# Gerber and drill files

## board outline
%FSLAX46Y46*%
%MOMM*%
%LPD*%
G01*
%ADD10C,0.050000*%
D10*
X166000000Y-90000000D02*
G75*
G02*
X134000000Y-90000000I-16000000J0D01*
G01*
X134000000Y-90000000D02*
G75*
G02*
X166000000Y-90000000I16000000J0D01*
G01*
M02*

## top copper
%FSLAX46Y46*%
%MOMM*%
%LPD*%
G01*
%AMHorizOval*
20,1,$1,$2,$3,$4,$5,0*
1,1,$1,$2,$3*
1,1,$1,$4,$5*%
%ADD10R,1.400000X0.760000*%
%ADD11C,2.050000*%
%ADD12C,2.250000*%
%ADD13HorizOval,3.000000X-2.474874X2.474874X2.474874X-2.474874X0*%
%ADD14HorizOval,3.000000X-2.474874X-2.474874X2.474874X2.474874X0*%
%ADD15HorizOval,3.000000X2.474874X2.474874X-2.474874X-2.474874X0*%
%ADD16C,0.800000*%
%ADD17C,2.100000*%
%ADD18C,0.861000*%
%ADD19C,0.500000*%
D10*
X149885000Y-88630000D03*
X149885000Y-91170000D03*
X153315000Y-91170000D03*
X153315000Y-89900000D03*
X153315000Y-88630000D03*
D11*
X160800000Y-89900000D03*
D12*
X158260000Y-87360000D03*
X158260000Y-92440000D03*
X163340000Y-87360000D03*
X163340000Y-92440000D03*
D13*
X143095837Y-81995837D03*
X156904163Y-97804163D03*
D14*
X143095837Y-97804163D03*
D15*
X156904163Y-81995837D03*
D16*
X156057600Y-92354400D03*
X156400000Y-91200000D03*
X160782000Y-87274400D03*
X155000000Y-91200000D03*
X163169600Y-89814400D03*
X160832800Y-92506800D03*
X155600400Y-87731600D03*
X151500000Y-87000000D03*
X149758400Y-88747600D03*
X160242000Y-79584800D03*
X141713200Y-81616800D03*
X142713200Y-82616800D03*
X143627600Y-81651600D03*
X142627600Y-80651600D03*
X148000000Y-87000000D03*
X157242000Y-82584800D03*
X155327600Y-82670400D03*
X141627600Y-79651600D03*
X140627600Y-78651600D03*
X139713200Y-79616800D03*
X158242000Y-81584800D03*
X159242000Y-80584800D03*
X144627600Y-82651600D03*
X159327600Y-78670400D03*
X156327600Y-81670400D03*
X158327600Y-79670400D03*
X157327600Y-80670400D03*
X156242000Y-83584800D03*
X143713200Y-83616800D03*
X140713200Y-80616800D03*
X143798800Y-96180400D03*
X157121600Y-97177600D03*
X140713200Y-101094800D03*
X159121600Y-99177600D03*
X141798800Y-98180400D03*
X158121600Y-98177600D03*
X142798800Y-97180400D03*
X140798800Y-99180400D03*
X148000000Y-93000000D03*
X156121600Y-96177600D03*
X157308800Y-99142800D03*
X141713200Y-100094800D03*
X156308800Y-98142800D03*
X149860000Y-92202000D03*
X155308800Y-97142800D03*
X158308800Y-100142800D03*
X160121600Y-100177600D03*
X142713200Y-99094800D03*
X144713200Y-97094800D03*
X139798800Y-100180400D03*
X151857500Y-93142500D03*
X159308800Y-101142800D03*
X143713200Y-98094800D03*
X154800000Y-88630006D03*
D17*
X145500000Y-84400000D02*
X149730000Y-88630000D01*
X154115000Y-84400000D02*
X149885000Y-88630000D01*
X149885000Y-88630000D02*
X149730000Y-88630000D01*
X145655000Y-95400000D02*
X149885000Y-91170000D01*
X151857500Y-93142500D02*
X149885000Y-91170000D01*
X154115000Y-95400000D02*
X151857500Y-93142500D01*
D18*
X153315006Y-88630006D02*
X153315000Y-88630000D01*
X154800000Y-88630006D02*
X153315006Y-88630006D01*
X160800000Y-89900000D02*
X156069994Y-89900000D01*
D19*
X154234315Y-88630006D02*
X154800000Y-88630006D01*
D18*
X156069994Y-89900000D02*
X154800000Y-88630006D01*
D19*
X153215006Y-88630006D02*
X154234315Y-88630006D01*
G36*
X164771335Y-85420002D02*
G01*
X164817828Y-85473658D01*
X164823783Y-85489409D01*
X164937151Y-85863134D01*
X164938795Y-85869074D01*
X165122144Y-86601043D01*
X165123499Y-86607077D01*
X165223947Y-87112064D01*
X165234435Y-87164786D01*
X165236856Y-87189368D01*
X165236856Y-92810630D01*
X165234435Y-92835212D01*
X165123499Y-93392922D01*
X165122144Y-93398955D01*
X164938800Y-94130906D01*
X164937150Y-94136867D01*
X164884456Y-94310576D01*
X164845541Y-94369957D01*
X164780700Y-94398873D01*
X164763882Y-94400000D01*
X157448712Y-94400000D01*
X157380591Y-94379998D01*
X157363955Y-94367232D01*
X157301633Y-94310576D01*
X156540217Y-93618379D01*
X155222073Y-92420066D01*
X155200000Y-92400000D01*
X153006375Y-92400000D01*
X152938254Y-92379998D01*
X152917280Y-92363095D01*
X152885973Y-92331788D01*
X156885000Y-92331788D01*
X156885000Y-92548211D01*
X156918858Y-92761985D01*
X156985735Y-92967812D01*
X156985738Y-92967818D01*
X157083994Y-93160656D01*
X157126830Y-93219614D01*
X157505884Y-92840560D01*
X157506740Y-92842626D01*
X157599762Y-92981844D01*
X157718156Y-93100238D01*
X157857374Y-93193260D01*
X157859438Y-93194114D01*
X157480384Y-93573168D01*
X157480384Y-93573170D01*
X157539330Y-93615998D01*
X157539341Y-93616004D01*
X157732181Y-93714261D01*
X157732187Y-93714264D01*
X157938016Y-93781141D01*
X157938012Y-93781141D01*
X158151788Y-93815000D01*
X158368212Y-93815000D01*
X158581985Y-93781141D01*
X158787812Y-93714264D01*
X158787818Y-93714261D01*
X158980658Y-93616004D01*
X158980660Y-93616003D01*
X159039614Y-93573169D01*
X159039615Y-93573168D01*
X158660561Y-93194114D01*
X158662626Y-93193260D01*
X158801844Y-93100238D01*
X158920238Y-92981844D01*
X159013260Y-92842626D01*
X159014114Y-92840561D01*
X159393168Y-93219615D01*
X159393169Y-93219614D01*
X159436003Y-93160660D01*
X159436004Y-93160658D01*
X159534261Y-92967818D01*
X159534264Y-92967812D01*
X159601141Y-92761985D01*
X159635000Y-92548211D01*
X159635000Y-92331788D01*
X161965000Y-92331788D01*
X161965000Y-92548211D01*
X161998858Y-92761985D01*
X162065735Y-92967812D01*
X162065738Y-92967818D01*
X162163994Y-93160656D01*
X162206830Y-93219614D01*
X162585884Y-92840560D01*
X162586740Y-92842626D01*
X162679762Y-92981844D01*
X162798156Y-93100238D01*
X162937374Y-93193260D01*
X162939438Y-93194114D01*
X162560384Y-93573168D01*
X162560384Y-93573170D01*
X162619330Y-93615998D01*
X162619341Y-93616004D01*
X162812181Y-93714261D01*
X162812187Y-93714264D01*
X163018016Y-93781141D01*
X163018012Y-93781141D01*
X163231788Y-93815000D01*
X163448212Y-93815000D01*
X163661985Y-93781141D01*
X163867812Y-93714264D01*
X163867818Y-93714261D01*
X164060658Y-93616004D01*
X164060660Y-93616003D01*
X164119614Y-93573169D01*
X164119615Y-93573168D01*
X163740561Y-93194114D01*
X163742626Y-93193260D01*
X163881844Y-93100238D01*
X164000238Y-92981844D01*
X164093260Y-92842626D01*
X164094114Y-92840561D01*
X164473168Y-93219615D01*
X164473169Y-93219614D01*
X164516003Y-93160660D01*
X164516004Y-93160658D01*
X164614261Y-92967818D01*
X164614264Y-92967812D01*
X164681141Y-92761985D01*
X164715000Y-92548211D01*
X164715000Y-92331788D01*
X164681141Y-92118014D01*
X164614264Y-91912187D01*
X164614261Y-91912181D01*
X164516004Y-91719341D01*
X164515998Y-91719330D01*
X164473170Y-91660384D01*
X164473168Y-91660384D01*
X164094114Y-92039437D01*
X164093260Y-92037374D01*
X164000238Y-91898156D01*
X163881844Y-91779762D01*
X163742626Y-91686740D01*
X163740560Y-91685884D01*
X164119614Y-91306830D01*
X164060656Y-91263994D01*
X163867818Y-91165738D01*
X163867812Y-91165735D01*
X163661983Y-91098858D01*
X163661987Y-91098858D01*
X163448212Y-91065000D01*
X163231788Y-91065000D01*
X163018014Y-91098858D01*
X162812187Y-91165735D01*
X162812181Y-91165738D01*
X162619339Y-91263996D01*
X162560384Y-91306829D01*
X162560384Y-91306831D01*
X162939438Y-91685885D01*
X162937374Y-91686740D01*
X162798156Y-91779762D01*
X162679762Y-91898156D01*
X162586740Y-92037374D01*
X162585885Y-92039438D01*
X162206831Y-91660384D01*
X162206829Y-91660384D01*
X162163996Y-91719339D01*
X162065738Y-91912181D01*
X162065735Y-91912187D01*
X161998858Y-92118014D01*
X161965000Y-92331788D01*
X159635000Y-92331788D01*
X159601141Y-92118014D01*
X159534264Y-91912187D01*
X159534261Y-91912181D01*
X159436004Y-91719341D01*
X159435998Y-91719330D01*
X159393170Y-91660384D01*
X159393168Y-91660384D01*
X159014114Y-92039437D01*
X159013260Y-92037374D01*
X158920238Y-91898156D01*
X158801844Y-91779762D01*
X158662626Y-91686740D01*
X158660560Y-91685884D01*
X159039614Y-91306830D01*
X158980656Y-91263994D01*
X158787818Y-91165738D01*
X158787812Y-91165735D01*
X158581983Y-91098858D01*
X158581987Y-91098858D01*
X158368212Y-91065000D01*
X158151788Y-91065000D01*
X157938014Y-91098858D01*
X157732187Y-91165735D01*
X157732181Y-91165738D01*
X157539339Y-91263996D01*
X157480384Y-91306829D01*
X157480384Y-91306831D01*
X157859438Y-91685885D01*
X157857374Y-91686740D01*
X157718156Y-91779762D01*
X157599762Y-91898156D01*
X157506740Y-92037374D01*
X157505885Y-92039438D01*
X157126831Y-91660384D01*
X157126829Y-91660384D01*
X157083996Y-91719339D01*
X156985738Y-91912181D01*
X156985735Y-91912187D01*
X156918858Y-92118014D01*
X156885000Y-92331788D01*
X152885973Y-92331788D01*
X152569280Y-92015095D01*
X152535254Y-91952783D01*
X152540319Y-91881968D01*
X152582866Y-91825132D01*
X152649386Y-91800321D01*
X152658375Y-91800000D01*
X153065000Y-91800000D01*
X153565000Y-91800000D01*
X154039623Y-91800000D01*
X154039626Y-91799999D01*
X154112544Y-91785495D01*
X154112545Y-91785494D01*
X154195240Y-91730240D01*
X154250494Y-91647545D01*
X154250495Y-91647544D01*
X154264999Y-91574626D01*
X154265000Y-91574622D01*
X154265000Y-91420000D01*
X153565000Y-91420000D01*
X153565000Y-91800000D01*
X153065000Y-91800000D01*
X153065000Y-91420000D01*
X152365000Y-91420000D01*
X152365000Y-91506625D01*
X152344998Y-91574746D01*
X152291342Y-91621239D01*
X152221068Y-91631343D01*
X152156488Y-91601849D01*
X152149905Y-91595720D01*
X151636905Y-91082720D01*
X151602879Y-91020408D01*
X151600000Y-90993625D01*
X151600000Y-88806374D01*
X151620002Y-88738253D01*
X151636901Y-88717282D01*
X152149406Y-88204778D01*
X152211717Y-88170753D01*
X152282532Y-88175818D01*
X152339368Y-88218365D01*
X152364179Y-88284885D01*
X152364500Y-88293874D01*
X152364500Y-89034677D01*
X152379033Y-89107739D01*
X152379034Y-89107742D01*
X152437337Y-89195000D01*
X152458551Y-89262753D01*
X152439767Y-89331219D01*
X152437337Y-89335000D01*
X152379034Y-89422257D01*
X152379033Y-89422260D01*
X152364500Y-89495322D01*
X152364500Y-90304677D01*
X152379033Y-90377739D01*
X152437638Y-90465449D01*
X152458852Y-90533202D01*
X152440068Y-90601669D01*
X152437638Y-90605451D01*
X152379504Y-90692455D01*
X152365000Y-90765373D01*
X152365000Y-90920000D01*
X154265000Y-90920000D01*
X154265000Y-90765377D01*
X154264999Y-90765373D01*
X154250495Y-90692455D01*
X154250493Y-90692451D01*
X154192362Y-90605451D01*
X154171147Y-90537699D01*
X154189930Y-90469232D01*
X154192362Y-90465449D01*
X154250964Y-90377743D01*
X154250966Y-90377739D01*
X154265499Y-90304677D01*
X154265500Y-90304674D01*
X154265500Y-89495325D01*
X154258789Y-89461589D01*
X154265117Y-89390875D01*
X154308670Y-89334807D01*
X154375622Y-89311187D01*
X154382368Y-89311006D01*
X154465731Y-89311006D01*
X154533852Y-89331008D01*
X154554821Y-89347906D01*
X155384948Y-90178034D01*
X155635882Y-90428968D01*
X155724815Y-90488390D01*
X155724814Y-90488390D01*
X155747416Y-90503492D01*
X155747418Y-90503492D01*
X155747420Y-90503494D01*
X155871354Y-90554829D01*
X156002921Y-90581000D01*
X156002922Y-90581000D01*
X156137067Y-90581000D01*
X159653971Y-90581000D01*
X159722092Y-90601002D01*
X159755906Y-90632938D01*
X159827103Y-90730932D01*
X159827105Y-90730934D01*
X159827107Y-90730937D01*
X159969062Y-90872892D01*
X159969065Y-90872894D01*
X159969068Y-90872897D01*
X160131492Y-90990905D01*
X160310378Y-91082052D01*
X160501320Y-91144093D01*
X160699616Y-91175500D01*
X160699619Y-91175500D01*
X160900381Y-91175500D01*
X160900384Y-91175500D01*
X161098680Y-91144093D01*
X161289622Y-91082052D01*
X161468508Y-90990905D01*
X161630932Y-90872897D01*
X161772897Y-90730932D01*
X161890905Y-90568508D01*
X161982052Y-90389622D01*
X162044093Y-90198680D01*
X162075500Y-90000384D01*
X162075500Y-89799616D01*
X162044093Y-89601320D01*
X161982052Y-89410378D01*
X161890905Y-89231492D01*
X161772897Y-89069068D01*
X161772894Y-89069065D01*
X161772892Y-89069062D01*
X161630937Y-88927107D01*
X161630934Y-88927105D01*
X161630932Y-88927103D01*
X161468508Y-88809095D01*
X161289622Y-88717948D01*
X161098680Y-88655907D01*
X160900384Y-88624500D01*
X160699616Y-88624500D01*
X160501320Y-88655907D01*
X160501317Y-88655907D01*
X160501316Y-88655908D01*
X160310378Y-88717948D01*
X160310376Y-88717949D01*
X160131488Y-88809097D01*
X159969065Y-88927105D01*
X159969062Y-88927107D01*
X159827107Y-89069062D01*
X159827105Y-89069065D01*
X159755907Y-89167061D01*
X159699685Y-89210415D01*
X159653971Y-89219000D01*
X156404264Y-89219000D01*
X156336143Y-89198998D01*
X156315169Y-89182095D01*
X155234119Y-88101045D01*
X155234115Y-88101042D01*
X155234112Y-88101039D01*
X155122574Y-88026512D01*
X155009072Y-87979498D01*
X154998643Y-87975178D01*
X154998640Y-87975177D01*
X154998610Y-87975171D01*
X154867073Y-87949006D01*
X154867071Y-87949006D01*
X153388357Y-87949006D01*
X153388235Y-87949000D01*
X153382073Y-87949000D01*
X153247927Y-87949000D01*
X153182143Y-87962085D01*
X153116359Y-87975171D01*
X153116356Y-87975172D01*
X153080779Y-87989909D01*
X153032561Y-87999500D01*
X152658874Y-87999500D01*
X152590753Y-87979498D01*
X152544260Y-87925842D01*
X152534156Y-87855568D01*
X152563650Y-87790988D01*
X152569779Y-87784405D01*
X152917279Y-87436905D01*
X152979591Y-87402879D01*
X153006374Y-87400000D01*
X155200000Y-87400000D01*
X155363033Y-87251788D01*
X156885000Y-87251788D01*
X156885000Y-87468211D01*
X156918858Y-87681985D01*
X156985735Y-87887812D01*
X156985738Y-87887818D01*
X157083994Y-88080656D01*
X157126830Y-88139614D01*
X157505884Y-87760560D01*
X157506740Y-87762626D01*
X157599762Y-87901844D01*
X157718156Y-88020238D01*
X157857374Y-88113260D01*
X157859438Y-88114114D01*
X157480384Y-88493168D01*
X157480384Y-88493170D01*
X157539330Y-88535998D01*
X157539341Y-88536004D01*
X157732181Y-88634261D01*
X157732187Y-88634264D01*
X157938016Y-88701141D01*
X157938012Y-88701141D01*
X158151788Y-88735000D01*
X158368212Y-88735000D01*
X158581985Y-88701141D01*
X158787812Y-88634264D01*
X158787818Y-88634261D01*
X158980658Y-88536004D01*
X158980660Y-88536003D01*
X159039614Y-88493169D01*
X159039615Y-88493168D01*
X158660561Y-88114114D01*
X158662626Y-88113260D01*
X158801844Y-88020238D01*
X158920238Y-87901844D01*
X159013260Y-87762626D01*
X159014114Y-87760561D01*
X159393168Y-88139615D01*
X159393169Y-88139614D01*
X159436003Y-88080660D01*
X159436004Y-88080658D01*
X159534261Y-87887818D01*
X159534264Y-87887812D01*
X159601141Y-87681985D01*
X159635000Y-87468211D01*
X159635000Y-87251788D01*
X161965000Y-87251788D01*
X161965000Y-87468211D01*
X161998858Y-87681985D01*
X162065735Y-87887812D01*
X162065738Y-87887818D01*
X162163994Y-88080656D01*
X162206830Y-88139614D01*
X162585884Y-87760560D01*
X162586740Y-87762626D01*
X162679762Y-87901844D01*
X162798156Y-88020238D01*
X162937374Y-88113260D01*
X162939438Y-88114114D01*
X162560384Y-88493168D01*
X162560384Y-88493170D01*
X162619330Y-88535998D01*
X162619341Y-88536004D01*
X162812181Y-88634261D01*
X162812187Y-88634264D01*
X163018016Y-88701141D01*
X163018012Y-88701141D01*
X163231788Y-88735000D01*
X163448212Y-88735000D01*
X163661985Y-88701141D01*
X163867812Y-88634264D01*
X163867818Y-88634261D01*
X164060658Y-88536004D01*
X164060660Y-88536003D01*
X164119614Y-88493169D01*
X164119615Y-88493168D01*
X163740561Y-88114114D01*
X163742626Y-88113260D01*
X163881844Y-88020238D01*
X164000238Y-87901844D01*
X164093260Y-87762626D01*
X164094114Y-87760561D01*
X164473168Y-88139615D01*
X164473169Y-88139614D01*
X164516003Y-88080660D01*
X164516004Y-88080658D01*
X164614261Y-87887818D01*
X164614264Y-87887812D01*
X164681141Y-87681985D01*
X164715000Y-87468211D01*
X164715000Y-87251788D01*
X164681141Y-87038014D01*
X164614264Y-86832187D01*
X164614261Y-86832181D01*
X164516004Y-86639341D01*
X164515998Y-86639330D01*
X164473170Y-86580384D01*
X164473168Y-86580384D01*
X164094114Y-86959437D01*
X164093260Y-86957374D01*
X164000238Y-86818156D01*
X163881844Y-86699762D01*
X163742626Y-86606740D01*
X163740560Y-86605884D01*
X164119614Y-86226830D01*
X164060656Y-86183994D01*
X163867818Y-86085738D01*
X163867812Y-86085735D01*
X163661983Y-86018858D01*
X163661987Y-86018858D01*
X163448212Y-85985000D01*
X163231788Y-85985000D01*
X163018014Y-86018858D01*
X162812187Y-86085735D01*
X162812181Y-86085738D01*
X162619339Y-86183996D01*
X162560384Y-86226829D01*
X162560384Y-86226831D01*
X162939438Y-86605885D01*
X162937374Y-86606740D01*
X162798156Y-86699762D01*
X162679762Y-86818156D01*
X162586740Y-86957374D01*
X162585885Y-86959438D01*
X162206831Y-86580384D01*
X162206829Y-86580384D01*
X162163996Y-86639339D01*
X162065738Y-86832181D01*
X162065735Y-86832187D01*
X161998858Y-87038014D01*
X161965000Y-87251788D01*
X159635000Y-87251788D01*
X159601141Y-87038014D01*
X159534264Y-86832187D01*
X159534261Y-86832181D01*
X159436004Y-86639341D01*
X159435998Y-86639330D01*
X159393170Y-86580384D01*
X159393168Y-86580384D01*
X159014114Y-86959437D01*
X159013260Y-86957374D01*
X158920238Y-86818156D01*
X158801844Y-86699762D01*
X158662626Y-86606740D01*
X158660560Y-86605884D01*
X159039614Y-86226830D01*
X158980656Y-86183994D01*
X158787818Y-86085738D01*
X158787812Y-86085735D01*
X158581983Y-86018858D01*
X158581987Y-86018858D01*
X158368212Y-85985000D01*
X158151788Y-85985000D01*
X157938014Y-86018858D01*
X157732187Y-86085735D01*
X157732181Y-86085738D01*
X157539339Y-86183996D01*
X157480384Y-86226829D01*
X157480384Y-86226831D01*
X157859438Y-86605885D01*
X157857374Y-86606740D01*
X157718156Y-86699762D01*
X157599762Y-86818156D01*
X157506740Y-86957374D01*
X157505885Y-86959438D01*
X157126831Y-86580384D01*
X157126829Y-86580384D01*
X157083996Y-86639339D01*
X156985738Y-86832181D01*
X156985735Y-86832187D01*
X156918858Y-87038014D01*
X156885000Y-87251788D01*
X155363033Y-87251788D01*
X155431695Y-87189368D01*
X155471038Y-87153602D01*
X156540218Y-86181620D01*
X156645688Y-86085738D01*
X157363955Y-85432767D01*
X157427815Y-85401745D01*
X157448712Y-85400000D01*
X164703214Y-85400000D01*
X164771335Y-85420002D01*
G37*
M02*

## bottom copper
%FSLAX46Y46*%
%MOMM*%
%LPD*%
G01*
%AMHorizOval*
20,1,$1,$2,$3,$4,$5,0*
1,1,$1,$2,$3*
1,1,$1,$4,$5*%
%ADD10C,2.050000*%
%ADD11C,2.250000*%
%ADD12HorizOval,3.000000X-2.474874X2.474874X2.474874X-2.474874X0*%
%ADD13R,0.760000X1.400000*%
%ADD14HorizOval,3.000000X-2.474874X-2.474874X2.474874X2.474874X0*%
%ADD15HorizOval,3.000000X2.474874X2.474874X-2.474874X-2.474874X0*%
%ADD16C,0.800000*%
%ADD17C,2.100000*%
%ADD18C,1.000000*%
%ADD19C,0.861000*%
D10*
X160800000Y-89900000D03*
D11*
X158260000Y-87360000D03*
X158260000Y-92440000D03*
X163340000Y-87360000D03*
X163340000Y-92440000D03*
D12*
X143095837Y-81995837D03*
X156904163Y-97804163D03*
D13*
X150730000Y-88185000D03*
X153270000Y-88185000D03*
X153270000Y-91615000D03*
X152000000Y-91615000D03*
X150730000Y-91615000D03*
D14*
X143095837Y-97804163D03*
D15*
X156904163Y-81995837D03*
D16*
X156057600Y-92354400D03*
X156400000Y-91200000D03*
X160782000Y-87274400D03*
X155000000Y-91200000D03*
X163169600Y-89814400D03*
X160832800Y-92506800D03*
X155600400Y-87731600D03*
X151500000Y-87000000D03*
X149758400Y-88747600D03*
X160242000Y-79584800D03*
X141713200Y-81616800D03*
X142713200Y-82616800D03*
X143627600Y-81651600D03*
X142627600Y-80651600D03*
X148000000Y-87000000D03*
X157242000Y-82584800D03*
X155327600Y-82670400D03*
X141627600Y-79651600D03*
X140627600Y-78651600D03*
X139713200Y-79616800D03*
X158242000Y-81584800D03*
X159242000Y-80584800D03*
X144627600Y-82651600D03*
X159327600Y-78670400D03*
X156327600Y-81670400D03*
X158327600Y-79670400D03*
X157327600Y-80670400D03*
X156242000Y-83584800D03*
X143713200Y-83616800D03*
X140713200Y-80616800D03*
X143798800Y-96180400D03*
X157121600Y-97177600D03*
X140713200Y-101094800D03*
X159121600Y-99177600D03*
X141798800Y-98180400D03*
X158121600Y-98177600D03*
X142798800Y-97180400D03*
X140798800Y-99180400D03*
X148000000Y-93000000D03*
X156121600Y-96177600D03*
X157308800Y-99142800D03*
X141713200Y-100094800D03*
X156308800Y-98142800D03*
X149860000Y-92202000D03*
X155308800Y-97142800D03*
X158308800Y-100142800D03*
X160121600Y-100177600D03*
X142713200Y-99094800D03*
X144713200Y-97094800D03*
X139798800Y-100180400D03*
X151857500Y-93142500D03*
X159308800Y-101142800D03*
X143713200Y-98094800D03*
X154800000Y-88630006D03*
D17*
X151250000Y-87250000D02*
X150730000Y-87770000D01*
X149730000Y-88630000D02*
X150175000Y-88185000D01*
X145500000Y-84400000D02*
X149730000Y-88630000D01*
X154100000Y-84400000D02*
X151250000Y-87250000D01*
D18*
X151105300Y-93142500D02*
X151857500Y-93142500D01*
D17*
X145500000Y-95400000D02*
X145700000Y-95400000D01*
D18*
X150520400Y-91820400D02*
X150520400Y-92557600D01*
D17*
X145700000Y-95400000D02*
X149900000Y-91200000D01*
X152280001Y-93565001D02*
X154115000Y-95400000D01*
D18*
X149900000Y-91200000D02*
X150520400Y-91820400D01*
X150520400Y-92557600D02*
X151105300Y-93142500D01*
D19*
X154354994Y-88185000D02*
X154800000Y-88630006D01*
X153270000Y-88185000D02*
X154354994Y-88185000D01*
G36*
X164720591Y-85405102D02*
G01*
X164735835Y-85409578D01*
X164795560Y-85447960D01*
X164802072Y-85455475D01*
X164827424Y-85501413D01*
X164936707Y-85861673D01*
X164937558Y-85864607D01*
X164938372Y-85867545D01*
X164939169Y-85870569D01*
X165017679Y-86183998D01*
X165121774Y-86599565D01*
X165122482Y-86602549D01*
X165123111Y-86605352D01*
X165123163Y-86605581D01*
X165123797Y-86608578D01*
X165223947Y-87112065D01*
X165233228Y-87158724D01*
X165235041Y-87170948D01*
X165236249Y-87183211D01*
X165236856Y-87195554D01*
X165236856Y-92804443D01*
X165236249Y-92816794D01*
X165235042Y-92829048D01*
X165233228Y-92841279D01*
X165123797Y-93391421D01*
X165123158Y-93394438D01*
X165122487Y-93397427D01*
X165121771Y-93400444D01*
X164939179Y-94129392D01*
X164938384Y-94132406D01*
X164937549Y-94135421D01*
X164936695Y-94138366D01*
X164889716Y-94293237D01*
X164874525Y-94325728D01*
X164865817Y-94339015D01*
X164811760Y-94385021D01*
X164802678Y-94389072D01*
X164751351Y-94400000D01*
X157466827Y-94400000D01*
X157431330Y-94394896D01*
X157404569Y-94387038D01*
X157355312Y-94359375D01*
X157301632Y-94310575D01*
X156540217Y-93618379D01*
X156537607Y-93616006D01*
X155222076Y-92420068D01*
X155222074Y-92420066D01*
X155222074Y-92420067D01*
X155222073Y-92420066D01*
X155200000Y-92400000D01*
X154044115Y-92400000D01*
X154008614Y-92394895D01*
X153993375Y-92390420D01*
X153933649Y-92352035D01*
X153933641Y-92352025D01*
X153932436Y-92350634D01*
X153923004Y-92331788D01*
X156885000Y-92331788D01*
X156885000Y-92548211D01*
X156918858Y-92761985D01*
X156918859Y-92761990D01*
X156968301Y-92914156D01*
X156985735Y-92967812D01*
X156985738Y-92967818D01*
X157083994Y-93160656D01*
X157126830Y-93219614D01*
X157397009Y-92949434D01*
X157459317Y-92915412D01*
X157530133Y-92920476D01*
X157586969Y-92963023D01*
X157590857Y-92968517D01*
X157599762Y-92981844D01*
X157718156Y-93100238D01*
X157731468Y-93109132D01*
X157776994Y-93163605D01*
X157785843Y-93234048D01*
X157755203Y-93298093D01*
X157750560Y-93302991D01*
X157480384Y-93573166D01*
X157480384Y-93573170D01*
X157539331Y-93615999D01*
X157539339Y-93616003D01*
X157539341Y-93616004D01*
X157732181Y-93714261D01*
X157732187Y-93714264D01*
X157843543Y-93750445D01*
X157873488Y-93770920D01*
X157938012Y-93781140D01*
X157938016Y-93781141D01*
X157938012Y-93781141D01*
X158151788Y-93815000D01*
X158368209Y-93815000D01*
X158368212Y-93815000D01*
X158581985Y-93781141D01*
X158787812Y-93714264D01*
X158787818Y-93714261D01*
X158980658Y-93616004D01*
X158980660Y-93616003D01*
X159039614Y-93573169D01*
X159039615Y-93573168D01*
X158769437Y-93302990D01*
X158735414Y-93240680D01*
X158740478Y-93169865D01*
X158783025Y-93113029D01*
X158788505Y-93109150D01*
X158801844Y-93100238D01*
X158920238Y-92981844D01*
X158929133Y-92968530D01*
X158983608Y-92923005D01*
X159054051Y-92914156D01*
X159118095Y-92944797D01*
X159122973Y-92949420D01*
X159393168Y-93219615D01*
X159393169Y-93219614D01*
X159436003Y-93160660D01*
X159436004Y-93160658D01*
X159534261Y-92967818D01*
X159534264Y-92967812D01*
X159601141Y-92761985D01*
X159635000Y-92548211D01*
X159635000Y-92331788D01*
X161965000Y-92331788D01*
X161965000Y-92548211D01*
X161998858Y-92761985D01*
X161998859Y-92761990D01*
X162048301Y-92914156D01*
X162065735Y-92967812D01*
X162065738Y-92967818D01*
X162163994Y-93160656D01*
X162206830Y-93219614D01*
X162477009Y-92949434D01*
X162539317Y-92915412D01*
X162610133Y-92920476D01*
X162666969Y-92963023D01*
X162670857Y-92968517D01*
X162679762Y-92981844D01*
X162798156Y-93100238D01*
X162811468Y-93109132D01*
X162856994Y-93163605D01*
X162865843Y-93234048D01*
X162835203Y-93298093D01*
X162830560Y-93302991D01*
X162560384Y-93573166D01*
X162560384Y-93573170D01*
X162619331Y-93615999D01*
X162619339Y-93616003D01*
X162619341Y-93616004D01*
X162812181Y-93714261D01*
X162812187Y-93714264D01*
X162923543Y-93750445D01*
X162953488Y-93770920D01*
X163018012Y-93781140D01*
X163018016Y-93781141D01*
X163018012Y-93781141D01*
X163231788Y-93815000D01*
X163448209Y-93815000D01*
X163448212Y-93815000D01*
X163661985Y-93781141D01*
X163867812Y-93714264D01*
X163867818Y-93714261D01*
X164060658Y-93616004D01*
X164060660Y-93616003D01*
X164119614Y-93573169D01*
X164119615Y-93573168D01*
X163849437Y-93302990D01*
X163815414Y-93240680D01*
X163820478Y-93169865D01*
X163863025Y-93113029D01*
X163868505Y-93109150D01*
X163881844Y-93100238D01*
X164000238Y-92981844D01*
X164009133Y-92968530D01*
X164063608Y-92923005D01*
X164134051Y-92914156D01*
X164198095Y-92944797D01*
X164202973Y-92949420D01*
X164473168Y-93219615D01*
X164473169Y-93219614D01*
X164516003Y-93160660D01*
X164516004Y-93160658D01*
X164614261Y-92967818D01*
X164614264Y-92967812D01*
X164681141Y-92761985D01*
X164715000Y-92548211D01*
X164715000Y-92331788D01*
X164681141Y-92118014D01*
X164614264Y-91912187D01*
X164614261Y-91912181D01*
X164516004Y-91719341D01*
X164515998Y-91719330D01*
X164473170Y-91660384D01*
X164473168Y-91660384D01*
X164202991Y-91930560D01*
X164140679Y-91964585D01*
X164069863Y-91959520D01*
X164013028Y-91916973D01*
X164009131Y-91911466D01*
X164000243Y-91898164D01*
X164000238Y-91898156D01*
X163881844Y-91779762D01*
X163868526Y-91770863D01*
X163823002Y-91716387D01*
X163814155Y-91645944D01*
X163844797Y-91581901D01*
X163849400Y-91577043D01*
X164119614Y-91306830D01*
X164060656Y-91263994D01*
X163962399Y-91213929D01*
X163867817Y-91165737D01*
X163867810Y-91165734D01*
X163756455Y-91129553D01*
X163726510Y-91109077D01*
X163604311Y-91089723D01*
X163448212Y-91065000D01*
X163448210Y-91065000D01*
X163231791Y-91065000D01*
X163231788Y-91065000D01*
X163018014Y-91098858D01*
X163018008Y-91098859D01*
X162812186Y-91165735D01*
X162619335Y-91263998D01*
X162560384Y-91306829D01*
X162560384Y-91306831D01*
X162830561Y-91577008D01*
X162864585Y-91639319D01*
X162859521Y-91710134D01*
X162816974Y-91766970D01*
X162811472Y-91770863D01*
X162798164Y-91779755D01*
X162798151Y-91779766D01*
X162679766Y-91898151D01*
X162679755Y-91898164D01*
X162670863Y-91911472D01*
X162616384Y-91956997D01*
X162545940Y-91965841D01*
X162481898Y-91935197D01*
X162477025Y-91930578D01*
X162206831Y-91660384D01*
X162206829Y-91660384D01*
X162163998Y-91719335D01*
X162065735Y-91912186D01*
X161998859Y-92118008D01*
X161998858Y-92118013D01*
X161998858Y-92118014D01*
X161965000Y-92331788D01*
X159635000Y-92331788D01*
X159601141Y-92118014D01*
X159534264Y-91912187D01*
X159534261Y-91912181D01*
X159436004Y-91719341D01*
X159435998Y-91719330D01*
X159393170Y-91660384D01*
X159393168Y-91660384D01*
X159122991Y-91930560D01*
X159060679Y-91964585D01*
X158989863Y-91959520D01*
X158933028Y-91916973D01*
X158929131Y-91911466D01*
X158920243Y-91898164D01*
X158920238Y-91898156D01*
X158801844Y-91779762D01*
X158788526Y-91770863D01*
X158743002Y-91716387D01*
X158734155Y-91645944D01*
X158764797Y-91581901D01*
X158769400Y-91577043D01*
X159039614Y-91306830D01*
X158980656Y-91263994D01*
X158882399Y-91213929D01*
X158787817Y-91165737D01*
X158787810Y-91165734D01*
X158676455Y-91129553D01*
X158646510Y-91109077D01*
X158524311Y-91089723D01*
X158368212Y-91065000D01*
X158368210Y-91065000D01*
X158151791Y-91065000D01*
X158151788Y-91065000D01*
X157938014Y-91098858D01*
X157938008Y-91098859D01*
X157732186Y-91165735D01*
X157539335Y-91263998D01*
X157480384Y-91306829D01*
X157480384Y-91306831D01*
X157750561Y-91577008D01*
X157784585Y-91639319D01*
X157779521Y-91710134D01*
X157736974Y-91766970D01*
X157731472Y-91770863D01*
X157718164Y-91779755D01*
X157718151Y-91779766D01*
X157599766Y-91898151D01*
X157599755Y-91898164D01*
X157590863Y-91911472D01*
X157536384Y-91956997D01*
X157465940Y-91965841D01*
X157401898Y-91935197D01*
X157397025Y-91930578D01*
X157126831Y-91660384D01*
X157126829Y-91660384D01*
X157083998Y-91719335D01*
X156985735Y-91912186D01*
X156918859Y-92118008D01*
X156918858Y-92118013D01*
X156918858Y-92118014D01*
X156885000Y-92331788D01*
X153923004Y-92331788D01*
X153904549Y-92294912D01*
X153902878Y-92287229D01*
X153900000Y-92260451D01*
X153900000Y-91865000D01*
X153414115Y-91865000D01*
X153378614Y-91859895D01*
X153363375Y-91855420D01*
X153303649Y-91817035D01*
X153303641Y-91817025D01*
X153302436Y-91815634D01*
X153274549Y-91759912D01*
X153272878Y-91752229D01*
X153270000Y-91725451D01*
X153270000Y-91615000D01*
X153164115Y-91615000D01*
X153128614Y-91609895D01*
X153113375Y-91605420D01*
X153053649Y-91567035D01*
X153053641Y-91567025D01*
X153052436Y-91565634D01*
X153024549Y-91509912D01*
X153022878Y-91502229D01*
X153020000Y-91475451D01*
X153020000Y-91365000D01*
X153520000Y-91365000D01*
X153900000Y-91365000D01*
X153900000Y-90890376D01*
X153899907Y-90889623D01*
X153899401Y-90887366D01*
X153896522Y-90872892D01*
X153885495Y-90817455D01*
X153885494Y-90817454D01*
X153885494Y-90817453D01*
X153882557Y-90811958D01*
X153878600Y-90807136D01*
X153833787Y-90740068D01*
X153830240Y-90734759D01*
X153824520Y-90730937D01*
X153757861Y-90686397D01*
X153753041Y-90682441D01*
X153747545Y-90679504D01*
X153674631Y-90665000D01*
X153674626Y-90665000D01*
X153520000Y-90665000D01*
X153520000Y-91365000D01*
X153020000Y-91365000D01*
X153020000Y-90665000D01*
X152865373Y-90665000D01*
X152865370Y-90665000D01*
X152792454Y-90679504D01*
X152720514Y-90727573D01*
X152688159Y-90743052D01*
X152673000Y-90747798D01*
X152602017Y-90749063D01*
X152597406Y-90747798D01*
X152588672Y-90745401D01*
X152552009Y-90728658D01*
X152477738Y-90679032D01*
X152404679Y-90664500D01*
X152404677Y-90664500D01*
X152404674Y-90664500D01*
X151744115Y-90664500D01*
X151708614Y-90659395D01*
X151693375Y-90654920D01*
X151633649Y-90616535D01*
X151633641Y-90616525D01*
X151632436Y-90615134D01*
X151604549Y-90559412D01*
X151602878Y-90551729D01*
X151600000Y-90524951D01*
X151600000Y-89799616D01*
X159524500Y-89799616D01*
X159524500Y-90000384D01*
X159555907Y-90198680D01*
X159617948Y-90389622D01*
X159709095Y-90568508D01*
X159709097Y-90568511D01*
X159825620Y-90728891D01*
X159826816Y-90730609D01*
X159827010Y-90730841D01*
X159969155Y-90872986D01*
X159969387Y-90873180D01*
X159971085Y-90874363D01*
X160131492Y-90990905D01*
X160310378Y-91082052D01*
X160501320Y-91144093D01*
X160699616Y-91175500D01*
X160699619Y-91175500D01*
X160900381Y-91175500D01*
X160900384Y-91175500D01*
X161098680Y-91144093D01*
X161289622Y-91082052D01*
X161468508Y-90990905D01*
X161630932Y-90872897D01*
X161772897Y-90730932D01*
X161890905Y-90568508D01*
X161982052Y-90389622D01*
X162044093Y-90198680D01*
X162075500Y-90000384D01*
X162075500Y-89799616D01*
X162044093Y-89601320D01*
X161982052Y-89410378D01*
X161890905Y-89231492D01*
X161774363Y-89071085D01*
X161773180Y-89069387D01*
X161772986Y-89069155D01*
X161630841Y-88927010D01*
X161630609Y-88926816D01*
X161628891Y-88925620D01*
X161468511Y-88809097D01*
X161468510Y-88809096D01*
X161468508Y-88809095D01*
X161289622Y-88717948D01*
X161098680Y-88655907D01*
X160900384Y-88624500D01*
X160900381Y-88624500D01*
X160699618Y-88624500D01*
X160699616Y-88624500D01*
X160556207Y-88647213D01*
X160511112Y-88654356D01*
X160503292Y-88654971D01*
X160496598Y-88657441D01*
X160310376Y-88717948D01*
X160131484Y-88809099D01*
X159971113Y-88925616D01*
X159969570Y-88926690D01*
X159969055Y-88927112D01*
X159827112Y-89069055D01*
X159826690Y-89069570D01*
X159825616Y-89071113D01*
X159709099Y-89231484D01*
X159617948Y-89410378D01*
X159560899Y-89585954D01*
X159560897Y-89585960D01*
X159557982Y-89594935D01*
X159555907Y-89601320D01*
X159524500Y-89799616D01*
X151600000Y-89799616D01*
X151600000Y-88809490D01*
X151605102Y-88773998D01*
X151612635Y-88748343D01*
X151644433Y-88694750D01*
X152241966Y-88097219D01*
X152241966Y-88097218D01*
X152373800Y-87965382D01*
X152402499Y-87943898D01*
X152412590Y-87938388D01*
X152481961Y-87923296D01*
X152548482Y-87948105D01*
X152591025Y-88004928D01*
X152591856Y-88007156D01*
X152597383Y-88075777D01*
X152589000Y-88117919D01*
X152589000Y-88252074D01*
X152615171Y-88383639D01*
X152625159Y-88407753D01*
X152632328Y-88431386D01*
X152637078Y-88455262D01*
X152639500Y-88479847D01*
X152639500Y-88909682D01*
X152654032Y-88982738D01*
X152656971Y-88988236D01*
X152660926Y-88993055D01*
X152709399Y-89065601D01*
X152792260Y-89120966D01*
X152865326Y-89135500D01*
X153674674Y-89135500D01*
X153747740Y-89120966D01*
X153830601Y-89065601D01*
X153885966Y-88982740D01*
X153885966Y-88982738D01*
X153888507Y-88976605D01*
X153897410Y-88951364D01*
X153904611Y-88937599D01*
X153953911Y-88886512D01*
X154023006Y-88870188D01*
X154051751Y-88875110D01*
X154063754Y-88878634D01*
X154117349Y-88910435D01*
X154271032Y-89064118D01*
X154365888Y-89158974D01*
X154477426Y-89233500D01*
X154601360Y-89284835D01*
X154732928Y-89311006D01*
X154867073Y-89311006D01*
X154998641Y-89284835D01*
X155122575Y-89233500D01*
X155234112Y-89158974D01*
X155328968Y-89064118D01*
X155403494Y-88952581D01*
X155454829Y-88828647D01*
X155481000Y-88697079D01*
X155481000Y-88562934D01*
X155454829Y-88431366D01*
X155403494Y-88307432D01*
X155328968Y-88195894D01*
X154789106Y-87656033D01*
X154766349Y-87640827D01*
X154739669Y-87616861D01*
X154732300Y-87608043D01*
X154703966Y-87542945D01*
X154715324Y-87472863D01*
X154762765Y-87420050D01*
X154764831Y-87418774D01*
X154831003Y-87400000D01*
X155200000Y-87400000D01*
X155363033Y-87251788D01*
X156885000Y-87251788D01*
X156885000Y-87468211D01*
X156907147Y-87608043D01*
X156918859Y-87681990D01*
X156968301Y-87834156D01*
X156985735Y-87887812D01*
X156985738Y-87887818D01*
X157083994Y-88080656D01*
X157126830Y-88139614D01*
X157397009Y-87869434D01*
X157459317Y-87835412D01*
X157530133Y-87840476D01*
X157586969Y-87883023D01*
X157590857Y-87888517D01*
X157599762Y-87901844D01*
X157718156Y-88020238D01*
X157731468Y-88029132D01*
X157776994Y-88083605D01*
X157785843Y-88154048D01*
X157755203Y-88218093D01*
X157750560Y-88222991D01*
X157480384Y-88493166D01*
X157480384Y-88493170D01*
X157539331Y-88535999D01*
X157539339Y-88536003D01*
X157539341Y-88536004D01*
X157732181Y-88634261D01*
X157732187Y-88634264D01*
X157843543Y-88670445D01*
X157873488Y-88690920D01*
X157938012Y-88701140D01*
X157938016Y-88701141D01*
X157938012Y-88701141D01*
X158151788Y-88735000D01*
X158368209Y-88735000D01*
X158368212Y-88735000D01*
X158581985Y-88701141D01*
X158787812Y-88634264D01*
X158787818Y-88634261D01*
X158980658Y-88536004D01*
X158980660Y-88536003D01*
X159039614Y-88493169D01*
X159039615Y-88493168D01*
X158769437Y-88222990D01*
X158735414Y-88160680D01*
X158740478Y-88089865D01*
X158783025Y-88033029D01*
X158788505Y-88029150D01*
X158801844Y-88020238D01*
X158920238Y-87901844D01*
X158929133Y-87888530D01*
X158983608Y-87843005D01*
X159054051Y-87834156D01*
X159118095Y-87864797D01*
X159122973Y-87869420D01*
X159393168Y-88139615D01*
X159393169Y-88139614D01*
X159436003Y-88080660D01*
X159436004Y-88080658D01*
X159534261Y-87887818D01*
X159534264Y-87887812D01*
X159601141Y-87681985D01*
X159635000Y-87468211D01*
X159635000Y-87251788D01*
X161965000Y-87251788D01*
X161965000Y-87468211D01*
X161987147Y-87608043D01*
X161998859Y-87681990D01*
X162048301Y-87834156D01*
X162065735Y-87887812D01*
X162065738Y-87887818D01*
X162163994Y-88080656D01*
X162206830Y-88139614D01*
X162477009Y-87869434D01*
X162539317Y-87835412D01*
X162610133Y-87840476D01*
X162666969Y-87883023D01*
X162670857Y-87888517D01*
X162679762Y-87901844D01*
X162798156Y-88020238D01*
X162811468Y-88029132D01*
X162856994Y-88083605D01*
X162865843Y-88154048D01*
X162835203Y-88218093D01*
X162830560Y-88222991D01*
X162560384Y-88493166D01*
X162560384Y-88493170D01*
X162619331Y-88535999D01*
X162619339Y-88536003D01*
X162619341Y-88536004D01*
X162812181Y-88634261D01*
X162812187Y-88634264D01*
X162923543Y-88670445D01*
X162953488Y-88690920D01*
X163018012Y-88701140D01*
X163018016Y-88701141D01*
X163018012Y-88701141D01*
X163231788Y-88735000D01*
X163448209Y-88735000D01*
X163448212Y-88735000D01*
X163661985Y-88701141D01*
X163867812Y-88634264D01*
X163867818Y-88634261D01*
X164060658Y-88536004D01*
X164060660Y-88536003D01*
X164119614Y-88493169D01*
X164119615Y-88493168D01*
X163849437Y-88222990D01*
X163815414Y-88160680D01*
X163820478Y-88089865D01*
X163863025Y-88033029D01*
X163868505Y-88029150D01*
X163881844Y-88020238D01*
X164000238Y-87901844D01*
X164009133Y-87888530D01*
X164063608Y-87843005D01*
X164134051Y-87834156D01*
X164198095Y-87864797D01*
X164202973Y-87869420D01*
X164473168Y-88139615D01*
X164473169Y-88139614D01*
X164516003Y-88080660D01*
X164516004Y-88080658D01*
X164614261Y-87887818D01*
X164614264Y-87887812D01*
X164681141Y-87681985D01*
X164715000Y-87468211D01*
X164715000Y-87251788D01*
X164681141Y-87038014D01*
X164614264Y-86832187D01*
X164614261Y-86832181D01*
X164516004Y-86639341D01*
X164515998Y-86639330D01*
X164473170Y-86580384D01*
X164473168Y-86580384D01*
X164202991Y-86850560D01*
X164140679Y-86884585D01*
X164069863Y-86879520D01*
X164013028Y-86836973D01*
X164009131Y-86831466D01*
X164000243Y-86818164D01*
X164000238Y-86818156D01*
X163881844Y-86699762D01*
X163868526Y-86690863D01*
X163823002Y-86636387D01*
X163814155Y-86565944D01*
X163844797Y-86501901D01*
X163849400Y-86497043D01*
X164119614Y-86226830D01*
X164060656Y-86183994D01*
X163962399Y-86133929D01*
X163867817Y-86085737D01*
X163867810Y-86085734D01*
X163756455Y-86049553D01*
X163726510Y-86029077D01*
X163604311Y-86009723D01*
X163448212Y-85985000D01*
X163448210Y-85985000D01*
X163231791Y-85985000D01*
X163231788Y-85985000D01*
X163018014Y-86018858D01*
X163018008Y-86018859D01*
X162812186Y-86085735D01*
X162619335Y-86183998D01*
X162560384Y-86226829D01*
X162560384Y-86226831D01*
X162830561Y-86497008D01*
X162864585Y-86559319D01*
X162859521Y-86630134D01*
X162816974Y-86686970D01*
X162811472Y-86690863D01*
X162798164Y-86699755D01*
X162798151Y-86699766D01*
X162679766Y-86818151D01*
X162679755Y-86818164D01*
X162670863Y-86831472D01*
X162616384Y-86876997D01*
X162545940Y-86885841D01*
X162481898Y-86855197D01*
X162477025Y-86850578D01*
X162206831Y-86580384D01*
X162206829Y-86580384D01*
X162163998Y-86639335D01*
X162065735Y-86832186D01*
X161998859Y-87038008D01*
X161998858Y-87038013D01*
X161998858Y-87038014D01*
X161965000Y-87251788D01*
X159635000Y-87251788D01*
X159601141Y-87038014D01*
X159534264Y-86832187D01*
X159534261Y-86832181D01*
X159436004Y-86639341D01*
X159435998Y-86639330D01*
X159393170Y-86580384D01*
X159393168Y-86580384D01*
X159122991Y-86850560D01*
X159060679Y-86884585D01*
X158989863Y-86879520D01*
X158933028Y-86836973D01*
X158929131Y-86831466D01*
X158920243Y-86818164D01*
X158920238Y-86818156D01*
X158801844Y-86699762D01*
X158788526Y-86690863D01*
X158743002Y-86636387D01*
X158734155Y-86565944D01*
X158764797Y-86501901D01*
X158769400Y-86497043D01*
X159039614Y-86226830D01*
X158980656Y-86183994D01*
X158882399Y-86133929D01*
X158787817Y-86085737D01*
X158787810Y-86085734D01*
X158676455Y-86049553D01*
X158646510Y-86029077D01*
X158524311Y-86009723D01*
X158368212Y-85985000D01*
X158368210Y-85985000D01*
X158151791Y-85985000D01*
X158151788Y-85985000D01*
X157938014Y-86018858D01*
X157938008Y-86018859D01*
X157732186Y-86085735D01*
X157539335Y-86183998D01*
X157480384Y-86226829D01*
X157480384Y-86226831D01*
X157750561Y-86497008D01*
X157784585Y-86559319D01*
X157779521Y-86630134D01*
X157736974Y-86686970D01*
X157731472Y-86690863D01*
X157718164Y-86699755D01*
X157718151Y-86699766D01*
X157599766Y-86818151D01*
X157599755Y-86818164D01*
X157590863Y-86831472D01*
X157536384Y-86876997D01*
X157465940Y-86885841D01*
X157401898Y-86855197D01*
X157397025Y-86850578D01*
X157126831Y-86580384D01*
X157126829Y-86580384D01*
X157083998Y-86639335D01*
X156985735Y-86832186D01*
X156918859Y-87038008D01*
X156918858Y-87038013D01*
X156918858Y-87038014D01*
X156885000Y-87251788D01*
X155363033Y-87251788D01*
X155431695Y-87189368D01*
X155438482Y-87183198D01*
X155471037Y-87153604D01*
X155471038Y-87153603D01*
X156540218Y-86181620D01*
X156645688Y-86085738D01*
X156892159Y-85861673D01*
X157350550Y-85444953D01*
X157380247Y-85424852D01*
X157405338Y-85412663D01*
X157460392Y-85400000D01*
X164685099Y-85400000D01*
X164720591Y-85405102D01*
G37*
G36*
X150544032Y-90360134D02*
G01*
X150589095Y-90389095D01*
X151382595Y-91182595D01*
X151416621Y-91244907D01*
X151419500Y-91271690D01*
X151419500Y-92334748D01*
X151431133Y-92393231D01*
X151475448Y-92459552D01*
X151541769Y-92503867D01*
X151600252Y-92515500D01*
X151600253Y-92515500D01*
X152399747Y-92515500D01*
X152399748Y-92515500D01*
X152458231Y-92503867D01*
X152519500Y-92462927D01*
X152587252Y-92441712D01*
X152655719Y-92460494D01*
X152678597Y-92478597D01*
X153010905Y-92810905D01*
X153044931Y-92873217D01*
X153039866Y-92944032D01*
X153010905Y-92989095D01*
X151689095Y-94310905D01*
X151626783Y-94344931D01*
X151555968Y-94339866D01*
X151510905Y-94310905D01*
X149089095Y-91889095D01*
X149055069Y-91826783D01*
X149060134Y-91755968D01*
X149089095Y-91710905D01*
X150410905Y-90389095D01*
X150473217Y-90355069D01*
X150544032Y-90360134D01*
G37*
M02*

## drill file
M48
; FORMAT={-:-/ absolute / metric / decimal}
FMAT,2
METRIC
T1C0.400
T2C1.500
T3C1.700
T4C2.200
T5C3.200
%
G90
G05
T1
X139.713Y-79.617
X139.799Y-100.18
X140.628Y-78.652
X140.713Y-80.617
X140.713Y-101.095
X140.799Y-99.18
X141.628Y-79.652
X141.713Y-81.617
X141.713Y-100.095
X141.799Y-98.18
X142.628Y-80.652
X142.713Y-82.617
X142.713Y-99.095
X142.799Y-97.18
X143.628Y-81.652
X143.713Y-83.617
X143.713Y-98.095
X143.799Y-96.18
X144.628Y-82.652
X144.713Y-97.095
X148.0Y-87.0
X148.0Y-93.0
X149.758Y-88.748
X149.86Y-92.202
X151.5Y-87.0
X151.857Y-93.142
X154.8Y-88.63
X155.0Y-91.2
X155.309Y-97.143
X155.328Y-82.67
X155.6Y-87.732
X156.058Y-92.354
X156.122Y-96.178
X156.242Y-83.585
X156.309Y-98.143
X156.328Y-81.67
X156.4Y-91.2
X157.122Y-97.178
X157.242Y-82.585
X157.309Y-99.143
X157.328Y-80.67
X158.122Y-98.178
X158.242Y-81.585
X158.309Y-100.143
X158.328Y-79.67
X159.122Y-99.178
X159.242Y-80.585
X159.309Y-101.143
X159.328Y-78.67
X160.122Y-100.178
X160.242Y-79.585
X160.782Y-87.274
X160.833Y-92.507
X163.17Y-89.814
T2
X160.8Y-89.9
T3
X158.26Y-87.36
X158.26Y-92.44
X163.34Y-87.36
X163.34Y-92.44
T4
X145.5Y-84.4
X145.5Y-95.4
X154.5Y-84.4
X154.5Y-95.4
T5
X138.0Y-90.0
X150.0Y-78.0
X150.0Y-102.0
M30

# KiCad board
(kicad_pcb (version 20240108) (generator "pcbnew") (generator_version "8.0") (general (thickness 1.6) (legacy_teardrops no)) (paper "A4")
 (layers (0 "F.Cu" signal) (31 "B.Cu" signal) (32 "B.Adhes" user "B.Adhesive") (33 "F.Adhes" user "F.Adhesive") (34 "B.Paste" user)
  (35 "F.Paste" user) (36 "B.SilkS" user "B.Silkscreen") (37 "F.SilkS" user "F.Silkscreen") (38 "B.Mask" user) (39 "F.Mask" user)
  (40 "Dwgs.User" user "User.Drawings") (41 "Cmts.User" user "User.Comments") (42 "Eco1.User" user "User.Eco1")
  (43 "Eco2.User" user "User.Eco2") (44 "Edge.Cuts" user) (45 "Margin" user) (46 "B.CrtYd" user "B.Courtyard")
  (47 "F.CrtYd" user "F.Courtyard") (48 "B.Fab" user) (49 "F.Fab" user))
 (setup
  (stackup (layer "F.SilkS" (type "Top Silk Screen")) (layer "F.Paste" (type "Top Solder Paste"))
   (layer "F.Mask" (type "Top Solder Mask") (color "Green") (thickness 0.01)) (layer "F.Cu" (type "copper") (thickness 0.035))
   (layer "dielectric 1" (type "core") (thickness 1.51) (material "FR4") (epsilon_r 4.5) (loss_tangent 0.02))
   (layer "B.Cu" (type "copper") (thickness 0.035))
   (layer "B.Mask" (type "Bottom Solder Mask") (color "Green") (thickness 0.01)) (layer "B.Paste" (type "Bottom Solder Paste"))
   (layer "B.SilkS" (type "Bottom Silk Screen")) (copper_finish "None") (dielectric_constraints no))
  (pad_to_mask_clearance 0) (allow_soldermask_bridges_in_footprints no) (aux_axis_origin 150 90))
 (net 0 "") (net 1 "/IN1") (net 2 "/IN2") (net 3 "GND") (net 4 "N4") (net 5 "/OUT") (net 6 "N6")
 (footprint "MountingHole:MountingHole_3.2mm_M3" (layer "F.Cu") (at 138 90)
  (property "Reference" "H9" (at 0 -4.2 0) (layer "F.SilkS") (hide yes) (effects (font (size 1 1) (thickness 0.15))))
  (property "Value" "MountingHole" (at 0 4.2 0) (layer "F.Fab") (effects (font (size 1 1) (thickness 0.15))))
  (pad "" np_thru_hole circle (at 0 0) (size 3.2 3.2) (drill 3.2) (layers "*.Cu" "*.Mask")))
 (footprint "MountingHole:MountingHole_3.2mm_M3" (layer "F.Cu") (at 150 102)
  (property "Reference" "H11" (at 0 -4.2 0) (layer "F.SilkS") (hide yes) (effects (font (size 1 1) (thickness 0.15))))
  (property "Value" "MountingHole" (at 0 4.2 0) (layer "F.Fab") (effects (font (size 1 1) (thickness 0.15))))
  (pad "" np_thru_hole circle (at 0 0) (size 3.2 3.2) (drill 3.2) (layers "*.Cu" "*.Mask")))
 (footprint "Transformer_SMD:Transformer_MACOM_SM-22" (layer "F.Cu") (at 151.6 89.9)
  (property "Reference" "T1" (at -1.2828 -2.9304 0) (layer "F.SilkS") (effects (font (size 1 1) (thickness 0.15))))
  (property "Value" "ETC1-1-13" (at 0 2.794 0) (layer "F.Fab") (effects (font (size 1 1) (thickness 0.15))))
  (pad "1" smd rect (at -1.715 -1.27) (size 1.4 0.76) (layers "F.Cu" "F.Paste" "F.Mask") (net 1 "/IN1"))
  (pad "2" smd rect (at -1.715 1.27) (size 1.4 0.76) (layers "F.Cu" "F.Paste" "F.Mask") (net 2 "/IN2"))
  (pad "3" smd rect (at 1.715 1.27) (size 1.4 0.76) (layers "F.Cu" "F.Paste" "F.Mask") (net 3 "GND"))
  (pad "4" smd rect (at 1.715 0) (size 1.4 0.76) (layers "F.Cu" "F.Paste" "F.Mask") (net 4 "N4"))
  (pad "5" smd rect (at 1.715 -1.27) (size 1.4 0.76) (layers "F.Cu" "F.Paste" "F.Mask") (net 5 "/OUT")))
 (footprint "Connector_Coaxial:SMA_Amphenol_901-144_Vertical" (layer "F.Cu") (at 160.8 89.9)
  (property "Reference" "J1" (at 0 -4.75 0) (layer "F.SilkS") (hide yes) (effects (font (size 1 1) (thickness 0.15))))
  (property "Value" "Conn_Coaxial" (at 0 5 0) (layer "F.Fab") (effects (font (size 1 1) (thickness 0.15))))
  (pad "1" thru_hole circle (at 0 0) (size 2.05 2.05) (drill 1.5) (layers "*.Cu" "*.Mask") (remove_unused_layers no) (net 5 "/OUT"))
  (pad "2" thru_hole circle (at -2.54 -2.54) (size 2.25 2.25) (drill 1.7) (layers "*.Cu" "*.Mask") (remove_unused_layers no) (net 3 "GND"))
  (pad "2" thru_hole circle (at -2.54 2.54) (size 2.25 2.25) (drill 1.7) (layers "*.Cu" "*.Mask") (remove_unused_layers no) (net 3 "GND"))
  (pad "2" thru_hole circle (at 2.54 -2.54) (size 2.25 2.25) (drill 1.7) (layers "*.Cu" "*.Mask") (remove_unused_layers no) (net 3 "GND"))
  (pad "2" thru_hole circle (at 2.54 2.54) (size 2.25 2.25) (drill 1.7) (layers "*.Cu" "*.Mask") (remove_unused_layers no) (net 3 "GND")))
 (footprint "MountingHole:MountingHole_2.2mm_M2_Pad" (layer "F.Cu") (at 145.5 84.4)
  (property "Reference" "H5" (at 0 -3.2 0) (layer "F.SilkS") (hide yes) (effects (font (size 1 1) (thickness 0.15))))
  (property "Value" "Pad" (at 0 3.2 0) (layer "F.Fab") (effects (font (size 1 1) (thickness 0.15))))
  (pad "1" thru_hole oval (at 0 0 45) (size 3 10) (drill 2.2 (offset 0 -3.4)) (layers "*.Cu" "*.Mask") (remove_unused_layers no)
   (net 1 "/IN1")))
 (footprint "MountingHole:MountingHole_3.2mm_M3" (layer "F.Cu") (at 150 78)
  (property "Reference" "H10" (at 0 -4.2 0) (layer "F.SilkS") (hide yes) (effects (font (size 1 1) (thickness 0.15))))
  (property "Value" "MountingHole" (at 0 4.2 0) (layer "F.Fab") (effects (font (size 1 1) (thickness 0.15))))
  (pad "" np_thru_hole circle (at 0 0) (size 3.2 3.2) (drill 3.2) (layers "*.Cu" "*.Mask")))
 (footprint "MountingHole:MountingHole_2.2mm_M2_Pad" (layer "F.Cu") (at 154.5 95.4 180)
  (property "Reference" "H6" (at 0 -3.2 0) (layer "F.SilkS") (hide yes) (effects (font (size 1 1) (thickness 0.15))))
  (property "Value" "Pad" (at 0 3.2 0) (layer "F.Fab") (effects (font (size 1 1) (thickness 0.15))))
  (pad "1" thru_hole oval (at 0 0 225) (size 3 10) (drill 2.2 (offset 0 -3.4)) (layers "*.Cu" "*.Mask") (remove_unused_layers no)
   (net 2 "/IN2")))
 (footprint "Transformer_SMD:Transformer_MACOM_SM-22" (layer "B.Cu") (at 152 89.9 -90)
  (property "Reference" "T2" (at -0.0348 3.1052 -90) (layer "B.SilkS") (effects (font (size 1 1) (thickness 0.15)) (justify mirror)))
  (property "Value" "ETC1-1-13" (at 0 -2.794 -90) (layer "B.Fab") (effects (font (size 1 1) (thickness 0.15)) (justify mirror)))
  (pad "1" smd rect (at -1.715 1.27 270) (size 1.4 0.76) (layers "B.Cu" "B.Paste" "B.Mask") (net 1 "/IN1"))
  (pad "2" smd rect (at -1.715 -1.27 270) (size 1.4 0.76) (layers "B.Cu" "B.Paste" "B.Mask") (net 5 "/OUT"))
  (pad "3" smd rect (at 1.715 -1.27 270) (size 1.4 0.76) (layers "B.Cu" "B.Paste" "B.Mask") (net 3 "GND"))
  (pad "4" smd rect (at 1.715 0 270) (size 1.4 0.76) (layers "B.Cu" "B.Paste" "B.Mask") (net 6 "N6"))
  (pad "5" smd rect (at 1.715 1.27 270) (size 1.4 0.76) (layers "B.Cu" "B.Paste" "B.Mask") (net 2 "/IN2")))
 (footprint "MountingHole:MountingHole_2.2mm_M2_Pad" (layer "B.Cu") (at 145.5 95.4)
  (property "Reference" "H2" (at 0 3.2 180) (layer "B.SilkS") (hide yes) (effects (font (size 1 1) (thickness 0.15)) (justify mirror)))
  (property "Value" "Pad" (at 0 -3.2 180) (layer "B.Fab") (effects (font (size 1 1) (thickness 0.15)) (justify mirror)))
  (pad "1" thru_hole oval (at 0 0 315) (size 3 10) (drill 2.2 (offset 0 3.4)) (layers "*.Cu" "*.Mask") (remove_unused_layers no)
   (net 2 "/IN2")))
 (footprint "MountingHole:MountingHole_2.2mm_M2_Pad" (layer "B.Cu") (at 154.5 84.4 180)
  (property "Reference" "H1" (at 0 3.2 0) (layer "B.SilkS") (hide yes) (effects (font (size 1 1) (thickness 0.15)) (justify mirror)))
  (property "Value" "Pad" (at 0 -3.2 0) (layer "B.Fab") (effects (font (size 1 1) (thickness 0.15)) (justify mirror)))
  (pad "1" thru_hole oval (at 0 0 135) (size 3 10) (drill 2.2 (offset 0 3.4)) (layers "*.Cu" "*.Mask") (remove_unused_layers yes)
   (keep_end_layers no) (zone_layer_connections) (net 1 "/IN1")))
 (gr_circle (center 150 90) (end 166 90) (stroke (width 0.05) (type solid)) (fill none) (layer "Edge.Cuts"))
 (via (at 156.0576 92.3544) (size 0.8) (drill 0.4) (layers "F.Cu" "B.Cu") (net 3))
 (via (at 156.4 91.2) (size 0.8) (drill 0.4) (layers "F.Cu" "B.Cu") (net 3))
 (via (at 160.782 87.2744) (size 0.8) (drill 0.4) (layers "F.Cu" "B.Cu") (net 3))
 (via (at 155 91.2) (size 0.8) (drill 0.4) (layers "F.Cu" "B.Cu") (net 3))
 (via (at 163.1696 89.8144) (size 0.8) (drill 0.4) (layers "F.Cu" "B.Cu") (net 3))
 (via (at 160.8328 92.5068) (size 0.8) (drill 0.4) (layers "F.Cu" "B.Cu") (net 3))
 (via (at 155.6004 87.7316) (size 0.8) (drill 0.4) (layers "F.Cu" "B.Cu") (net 3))
 (segment (start 145.5 84.4) (end 149.73 88.63) (width 2.1) (layer "F.Cu") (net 1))
 (segment (start 154.115 84.4) (end 149.885 88.63) (width 2.1) (layer "F.Cu") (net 1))
 (segment (start 149.885 88.63) (end 149.73 88.63) (width 2.1) (layer "F.Cu") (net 1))
 (via (at 151.5 87) (size 0.8) (drill 0.4) (layers "F.Cu" "B.Cu") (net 1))
 (via (at 149.7584 88.7476) (size 0.8) (drill 0.4) (layers "F.Cu" "B.Cu") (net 1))
 (via (at 160.242 79.5848) (size 0.8) (drill 0.4) (layers "F.Cu" "B.Cu") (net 1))
 (via (at 141.7132 81.6168) (size 0.8) (drill 0.4) (layers "F.Cu" "B.Cu") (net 1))
 (via (at 142.7132 82.6168) (size 0.8) (drill 0.4) (layers "F.Cu" "B.Cu") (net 1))
 (via (at 143.6276 81.6516) (size 0.8) (drill 0.4) (layers "F.Cu" "B.Cu") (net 1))
 (via (at 142.6276 80.6516) (size 0.8) (drill 0.4) (layers "F.Cu" "B.Cu") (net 1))
 (via (at 148 87) (size 0.8) (drill 0.4) (layers "F.Cu" "B.Cu") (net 1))
 (via (at 157.242 82.5848) (size 0.8) (drill 0.4) (layers "F.Cu" "B.Cu") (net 1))
 (via (at 155.3276 82.6704) (size 0.8) (drill 0.4) (layers "F.Cu" "B.Cu") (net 1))
 (via (at 141.6276 79.6516) (size 0.8) (drill 0.4) (layers "F.Cu" "B.Cu") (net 1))
 (via (at 140.6276 78.6516) (size 0.8) (drill 0.4) (layers "F.Cu" "B.Cu") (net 1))
 (via (at 139.7132 79.6168) (size 0.8) (drill 0.4) (layers "F.Cu" "B.Cu") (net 1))
 (via (at 158.242 81.5848) (size 0.8) (drill 0.4) (layers "F.Cu" "B.Cu") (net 1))
 (via (at 159.242 80.5848) (size 0.8) (drill 0.4) (layers "F.Cu" "B.Cu") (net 1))
 (via (at 144.6276 82.6516) (size 0.8) (drill 0.4) (layers "F.Cu" "B.Cu") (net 1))
 (via (at 159.3276 78.6704) (size 0.8) (drill 0.4) (layers "F.Cu" "B.Cu") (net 1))
 (via (at 156.3276 81.6704) (size 0.8) (drill 0.4) (layers "F.Cu" "B.Cu") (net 1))
 (via (at 158.3276 79.6704) (size 0.8) (drill 0.4) (layers "F.Cu" "B.Cu") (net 1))
 (via (at 157.3276 80.6704) (size 0.8) (drill 0.4) (layers "F.Cu" "B.Cu") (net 1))
 (via (at 156.242 83.5848) (size 0.8) (drill 0.4) (layers "F.Cu" "B.Cu") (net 1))
 (via (at 143.7132 83.6168) (size 0.8) (drill 0.4) (layers "F.Cu" "B.Cu") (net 1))
 (via (at 140.7132 80.6168) (size 0.8) (drill 0.4) (layers "F.Cu" "B.Cu") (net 1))
 (segment (start 151.25 87.25) (end 150.73 87.77) (width 2.1) (layer "B.Cu") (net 1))
 (segment (start 149.73 88.63) (end 150.175 88.185) (width 2.1) (layer "B.Cu") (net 1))
 (segment (start 145.5 84.4) (end 149.73 88.63) (width 2.1) (layer "B.Cu") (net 1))
 (segment (start 154.1 84.4) (end 151.25 87.25) (width 2.1) (layer "B.Cu") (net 1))
 (segment (start 145.655 95.4) (end 149.885 91.17) (width 2.1) (layer "F.Cu") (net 2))
 (segment (start 151.8575 93.1425) (end 149.885 91.17) (width 2.1) (layer "F.Cu") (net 2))
 (segment (start 154.115 95.4) (end 151.8575 93.1425) (width 2.1) (layer "F.Cu") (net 2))
 (via (at 143.7988 96.1804) (size 0.8) (drill 0.4) (layers "F.Cu" "B.Cu") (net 2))
 (via (at 157.1216 97.1776) (size 0.8) (drill 0.4) (layers "F.Cu" "B.Cu") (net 2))
 (via (at 140.7132 101.0948) (size 0.8) (drill 0.4) (layers "F.Cu" "B.Cu") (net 2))
 (via (at 159.1216 99.1776) (size 0.8) (drill 0.4) (layers "F.Cu" "B.Cu") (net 2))
 (via (at 141.7988 98.1804) (size 0.8) (drill 0.4) (layers "F.Cu" "B.Cu") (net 2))
 (via (at 158.1216 98.1776) (size 0.8) (drill 0.4) (layers "F.Cu" "B.Cu") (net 2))
 (via (at 142.7988 97.1804) (size 0.8) (drill 0.4) (layers "F.Cu" "B.Cu") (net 2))
 (via (at 140.7988 99.1804) (size 0.8) (drill 0.4) (layers "F.Cu" "B.Cu") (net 2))
 (via (at 148 93) (size 0.8) (drill 0.4) (layers "F.Cu" "B.Cu") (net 2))
 (via (at 156.1216 96.1776) (size 0.8) (drill 0.4) (layers "F.Cu" "B.Cu") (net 2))
 (via (at 157.3088 99.1428) (size 0.8) (drill 0.4) (layers "F.Cu" "B.Cu") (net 2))
 (via (at 141.7132 100.0948) (size 0.8) (drill 0.4) (layers "F.Cu" "B.Cu") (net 2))
 (via (at 156.3088 98.1428) (size 0.8) (drill 0.4) (layers "F.Cu" "B.Cu") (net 2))
 (via (at 149.86 92.202) (size 0.8) (drill 0.4) (layers "F.Cu" "B.Cu") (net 2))
 (via (at 155.3088 97.1428) (size 0.8) (drill 0.4) (layers "F.Cu" "B.Cu") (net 2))
 (via (at 158.3088 100.1428) (size 0.8) (drill 0.4) (layers "F.Cu" "B.Cu") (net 2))
 (via (at 160.1216 100.1776) (size 0.8) (drill 0.4) (layers "F.Cu" "B.Cu") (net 2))
 (via (at 142.7132 99.0948) (size 0.8) (drill 0.4) (layers "F.Cu" "B.Cu") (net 2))
 (via (at 144.7132 97.0948) (size 0.8) (drill 0.4) (layers "F.Cu" "B.Cu") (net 2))
 (via (at 139.7988 100.1804) (size 0.8) (drill 0.4) (layers "F.Cu" "B.Cu") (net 2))
 (via (at 151.8575 93.1425) (size 0.8) (drill 0.4) (layers "F.Cu" "B.Cu") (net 2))
 (via (at 159.3088 101.1428) (size 0.8) (drill 0.4) (layers "F.Cu" "B.Cu") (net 2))
 (via (at 143.7132 98.0948) (size 0.8) (drill 0.4) (layers "F.Cu" "B.Cu") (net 2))
 (segment (start 151.1053 93.1425) (end 151.8575 93.1425) (width 1) (layer "B.Cu") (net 2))
 (segment (start 145.5 95.4) (end 145.7 95.4) (width 2.1) (layer "B.Cu") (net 2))
 (segment (start 150.5204 91.8204) (end 150.5204 92.5576) (width 1) (layer "B.Cu") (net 2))
 (segment (start 145.7 95.4) (end 149.9 91.2) (width 2.1) (layer "B.Cu") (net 2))
 (segment (start 152.280001 93.565001) (end 154.115 95.4) (width 2.1) (layer "B.Cu") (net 2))
 (segment (start 149.9 91.2) (end 150.5204 91.8204) (width 1) (layer "B.Cu") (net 2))
 (segment (start 150.5204 92.5576) (end 151.1053 93.1425) (width 1) (layer "B.Cu") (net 2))
 (segment (start 153.315006 88.630006) (end 153.315 88.63) (width 0.861) (layer "F.Cu") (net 5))
 (segment (start 154.8 88.630006) (end 153.315006 88.630006) (width 0.861) (layer "F.Cu") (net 5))
 (segment (start 160.8 89.9) (end 156.069994 89.9) (width 0.861) (layer "F.Cu") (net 5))
 (segment (start 154.234315 88.630006) (end 154.8 88.630006) (width 0.5) (layer "F.Cu") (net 5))
 (segment (start 156.069994 89.9) (end 154.8 88.630006) (width 0.861) (layer "F.Cu") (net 5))
 (segment (start 153.215006 88.630006) (end 154.234315 88.630006) (width 0.5) (layer "F.Cu") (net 5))
 (via (at 154.8 88.630006) (size 0.8) (drill 0.4) (layers "F.Cu" "B.Cu") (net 5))
 (segment (start 154.354994 88.185) (end 154.8 88.630006) (width 0.861) (layer "B.Cu") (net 5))
 (segment (start 153.27 88.185) (end 154.354994 88.185) (width 0.861) (layer "B.Cu") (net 5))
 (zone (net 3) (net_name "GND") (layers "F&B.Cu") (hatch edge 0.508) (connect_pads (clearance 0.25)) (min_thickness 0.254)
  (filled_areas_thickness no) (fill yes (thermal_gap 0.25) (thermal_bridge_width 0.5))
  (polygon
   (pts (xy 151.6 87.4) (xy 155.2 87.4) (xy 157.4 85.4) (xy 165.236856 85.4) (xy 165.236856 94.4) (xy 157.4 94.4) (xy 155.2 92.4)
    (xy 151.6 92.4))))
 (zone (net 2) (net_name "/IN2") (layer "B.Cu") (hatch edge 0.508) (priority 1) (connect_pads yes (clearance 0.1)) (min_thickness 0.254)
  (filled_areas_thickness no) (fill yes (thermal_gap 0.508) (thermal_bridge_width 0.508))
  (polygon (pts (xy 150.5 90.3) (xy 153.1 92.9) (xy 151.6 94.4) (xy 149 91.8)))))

